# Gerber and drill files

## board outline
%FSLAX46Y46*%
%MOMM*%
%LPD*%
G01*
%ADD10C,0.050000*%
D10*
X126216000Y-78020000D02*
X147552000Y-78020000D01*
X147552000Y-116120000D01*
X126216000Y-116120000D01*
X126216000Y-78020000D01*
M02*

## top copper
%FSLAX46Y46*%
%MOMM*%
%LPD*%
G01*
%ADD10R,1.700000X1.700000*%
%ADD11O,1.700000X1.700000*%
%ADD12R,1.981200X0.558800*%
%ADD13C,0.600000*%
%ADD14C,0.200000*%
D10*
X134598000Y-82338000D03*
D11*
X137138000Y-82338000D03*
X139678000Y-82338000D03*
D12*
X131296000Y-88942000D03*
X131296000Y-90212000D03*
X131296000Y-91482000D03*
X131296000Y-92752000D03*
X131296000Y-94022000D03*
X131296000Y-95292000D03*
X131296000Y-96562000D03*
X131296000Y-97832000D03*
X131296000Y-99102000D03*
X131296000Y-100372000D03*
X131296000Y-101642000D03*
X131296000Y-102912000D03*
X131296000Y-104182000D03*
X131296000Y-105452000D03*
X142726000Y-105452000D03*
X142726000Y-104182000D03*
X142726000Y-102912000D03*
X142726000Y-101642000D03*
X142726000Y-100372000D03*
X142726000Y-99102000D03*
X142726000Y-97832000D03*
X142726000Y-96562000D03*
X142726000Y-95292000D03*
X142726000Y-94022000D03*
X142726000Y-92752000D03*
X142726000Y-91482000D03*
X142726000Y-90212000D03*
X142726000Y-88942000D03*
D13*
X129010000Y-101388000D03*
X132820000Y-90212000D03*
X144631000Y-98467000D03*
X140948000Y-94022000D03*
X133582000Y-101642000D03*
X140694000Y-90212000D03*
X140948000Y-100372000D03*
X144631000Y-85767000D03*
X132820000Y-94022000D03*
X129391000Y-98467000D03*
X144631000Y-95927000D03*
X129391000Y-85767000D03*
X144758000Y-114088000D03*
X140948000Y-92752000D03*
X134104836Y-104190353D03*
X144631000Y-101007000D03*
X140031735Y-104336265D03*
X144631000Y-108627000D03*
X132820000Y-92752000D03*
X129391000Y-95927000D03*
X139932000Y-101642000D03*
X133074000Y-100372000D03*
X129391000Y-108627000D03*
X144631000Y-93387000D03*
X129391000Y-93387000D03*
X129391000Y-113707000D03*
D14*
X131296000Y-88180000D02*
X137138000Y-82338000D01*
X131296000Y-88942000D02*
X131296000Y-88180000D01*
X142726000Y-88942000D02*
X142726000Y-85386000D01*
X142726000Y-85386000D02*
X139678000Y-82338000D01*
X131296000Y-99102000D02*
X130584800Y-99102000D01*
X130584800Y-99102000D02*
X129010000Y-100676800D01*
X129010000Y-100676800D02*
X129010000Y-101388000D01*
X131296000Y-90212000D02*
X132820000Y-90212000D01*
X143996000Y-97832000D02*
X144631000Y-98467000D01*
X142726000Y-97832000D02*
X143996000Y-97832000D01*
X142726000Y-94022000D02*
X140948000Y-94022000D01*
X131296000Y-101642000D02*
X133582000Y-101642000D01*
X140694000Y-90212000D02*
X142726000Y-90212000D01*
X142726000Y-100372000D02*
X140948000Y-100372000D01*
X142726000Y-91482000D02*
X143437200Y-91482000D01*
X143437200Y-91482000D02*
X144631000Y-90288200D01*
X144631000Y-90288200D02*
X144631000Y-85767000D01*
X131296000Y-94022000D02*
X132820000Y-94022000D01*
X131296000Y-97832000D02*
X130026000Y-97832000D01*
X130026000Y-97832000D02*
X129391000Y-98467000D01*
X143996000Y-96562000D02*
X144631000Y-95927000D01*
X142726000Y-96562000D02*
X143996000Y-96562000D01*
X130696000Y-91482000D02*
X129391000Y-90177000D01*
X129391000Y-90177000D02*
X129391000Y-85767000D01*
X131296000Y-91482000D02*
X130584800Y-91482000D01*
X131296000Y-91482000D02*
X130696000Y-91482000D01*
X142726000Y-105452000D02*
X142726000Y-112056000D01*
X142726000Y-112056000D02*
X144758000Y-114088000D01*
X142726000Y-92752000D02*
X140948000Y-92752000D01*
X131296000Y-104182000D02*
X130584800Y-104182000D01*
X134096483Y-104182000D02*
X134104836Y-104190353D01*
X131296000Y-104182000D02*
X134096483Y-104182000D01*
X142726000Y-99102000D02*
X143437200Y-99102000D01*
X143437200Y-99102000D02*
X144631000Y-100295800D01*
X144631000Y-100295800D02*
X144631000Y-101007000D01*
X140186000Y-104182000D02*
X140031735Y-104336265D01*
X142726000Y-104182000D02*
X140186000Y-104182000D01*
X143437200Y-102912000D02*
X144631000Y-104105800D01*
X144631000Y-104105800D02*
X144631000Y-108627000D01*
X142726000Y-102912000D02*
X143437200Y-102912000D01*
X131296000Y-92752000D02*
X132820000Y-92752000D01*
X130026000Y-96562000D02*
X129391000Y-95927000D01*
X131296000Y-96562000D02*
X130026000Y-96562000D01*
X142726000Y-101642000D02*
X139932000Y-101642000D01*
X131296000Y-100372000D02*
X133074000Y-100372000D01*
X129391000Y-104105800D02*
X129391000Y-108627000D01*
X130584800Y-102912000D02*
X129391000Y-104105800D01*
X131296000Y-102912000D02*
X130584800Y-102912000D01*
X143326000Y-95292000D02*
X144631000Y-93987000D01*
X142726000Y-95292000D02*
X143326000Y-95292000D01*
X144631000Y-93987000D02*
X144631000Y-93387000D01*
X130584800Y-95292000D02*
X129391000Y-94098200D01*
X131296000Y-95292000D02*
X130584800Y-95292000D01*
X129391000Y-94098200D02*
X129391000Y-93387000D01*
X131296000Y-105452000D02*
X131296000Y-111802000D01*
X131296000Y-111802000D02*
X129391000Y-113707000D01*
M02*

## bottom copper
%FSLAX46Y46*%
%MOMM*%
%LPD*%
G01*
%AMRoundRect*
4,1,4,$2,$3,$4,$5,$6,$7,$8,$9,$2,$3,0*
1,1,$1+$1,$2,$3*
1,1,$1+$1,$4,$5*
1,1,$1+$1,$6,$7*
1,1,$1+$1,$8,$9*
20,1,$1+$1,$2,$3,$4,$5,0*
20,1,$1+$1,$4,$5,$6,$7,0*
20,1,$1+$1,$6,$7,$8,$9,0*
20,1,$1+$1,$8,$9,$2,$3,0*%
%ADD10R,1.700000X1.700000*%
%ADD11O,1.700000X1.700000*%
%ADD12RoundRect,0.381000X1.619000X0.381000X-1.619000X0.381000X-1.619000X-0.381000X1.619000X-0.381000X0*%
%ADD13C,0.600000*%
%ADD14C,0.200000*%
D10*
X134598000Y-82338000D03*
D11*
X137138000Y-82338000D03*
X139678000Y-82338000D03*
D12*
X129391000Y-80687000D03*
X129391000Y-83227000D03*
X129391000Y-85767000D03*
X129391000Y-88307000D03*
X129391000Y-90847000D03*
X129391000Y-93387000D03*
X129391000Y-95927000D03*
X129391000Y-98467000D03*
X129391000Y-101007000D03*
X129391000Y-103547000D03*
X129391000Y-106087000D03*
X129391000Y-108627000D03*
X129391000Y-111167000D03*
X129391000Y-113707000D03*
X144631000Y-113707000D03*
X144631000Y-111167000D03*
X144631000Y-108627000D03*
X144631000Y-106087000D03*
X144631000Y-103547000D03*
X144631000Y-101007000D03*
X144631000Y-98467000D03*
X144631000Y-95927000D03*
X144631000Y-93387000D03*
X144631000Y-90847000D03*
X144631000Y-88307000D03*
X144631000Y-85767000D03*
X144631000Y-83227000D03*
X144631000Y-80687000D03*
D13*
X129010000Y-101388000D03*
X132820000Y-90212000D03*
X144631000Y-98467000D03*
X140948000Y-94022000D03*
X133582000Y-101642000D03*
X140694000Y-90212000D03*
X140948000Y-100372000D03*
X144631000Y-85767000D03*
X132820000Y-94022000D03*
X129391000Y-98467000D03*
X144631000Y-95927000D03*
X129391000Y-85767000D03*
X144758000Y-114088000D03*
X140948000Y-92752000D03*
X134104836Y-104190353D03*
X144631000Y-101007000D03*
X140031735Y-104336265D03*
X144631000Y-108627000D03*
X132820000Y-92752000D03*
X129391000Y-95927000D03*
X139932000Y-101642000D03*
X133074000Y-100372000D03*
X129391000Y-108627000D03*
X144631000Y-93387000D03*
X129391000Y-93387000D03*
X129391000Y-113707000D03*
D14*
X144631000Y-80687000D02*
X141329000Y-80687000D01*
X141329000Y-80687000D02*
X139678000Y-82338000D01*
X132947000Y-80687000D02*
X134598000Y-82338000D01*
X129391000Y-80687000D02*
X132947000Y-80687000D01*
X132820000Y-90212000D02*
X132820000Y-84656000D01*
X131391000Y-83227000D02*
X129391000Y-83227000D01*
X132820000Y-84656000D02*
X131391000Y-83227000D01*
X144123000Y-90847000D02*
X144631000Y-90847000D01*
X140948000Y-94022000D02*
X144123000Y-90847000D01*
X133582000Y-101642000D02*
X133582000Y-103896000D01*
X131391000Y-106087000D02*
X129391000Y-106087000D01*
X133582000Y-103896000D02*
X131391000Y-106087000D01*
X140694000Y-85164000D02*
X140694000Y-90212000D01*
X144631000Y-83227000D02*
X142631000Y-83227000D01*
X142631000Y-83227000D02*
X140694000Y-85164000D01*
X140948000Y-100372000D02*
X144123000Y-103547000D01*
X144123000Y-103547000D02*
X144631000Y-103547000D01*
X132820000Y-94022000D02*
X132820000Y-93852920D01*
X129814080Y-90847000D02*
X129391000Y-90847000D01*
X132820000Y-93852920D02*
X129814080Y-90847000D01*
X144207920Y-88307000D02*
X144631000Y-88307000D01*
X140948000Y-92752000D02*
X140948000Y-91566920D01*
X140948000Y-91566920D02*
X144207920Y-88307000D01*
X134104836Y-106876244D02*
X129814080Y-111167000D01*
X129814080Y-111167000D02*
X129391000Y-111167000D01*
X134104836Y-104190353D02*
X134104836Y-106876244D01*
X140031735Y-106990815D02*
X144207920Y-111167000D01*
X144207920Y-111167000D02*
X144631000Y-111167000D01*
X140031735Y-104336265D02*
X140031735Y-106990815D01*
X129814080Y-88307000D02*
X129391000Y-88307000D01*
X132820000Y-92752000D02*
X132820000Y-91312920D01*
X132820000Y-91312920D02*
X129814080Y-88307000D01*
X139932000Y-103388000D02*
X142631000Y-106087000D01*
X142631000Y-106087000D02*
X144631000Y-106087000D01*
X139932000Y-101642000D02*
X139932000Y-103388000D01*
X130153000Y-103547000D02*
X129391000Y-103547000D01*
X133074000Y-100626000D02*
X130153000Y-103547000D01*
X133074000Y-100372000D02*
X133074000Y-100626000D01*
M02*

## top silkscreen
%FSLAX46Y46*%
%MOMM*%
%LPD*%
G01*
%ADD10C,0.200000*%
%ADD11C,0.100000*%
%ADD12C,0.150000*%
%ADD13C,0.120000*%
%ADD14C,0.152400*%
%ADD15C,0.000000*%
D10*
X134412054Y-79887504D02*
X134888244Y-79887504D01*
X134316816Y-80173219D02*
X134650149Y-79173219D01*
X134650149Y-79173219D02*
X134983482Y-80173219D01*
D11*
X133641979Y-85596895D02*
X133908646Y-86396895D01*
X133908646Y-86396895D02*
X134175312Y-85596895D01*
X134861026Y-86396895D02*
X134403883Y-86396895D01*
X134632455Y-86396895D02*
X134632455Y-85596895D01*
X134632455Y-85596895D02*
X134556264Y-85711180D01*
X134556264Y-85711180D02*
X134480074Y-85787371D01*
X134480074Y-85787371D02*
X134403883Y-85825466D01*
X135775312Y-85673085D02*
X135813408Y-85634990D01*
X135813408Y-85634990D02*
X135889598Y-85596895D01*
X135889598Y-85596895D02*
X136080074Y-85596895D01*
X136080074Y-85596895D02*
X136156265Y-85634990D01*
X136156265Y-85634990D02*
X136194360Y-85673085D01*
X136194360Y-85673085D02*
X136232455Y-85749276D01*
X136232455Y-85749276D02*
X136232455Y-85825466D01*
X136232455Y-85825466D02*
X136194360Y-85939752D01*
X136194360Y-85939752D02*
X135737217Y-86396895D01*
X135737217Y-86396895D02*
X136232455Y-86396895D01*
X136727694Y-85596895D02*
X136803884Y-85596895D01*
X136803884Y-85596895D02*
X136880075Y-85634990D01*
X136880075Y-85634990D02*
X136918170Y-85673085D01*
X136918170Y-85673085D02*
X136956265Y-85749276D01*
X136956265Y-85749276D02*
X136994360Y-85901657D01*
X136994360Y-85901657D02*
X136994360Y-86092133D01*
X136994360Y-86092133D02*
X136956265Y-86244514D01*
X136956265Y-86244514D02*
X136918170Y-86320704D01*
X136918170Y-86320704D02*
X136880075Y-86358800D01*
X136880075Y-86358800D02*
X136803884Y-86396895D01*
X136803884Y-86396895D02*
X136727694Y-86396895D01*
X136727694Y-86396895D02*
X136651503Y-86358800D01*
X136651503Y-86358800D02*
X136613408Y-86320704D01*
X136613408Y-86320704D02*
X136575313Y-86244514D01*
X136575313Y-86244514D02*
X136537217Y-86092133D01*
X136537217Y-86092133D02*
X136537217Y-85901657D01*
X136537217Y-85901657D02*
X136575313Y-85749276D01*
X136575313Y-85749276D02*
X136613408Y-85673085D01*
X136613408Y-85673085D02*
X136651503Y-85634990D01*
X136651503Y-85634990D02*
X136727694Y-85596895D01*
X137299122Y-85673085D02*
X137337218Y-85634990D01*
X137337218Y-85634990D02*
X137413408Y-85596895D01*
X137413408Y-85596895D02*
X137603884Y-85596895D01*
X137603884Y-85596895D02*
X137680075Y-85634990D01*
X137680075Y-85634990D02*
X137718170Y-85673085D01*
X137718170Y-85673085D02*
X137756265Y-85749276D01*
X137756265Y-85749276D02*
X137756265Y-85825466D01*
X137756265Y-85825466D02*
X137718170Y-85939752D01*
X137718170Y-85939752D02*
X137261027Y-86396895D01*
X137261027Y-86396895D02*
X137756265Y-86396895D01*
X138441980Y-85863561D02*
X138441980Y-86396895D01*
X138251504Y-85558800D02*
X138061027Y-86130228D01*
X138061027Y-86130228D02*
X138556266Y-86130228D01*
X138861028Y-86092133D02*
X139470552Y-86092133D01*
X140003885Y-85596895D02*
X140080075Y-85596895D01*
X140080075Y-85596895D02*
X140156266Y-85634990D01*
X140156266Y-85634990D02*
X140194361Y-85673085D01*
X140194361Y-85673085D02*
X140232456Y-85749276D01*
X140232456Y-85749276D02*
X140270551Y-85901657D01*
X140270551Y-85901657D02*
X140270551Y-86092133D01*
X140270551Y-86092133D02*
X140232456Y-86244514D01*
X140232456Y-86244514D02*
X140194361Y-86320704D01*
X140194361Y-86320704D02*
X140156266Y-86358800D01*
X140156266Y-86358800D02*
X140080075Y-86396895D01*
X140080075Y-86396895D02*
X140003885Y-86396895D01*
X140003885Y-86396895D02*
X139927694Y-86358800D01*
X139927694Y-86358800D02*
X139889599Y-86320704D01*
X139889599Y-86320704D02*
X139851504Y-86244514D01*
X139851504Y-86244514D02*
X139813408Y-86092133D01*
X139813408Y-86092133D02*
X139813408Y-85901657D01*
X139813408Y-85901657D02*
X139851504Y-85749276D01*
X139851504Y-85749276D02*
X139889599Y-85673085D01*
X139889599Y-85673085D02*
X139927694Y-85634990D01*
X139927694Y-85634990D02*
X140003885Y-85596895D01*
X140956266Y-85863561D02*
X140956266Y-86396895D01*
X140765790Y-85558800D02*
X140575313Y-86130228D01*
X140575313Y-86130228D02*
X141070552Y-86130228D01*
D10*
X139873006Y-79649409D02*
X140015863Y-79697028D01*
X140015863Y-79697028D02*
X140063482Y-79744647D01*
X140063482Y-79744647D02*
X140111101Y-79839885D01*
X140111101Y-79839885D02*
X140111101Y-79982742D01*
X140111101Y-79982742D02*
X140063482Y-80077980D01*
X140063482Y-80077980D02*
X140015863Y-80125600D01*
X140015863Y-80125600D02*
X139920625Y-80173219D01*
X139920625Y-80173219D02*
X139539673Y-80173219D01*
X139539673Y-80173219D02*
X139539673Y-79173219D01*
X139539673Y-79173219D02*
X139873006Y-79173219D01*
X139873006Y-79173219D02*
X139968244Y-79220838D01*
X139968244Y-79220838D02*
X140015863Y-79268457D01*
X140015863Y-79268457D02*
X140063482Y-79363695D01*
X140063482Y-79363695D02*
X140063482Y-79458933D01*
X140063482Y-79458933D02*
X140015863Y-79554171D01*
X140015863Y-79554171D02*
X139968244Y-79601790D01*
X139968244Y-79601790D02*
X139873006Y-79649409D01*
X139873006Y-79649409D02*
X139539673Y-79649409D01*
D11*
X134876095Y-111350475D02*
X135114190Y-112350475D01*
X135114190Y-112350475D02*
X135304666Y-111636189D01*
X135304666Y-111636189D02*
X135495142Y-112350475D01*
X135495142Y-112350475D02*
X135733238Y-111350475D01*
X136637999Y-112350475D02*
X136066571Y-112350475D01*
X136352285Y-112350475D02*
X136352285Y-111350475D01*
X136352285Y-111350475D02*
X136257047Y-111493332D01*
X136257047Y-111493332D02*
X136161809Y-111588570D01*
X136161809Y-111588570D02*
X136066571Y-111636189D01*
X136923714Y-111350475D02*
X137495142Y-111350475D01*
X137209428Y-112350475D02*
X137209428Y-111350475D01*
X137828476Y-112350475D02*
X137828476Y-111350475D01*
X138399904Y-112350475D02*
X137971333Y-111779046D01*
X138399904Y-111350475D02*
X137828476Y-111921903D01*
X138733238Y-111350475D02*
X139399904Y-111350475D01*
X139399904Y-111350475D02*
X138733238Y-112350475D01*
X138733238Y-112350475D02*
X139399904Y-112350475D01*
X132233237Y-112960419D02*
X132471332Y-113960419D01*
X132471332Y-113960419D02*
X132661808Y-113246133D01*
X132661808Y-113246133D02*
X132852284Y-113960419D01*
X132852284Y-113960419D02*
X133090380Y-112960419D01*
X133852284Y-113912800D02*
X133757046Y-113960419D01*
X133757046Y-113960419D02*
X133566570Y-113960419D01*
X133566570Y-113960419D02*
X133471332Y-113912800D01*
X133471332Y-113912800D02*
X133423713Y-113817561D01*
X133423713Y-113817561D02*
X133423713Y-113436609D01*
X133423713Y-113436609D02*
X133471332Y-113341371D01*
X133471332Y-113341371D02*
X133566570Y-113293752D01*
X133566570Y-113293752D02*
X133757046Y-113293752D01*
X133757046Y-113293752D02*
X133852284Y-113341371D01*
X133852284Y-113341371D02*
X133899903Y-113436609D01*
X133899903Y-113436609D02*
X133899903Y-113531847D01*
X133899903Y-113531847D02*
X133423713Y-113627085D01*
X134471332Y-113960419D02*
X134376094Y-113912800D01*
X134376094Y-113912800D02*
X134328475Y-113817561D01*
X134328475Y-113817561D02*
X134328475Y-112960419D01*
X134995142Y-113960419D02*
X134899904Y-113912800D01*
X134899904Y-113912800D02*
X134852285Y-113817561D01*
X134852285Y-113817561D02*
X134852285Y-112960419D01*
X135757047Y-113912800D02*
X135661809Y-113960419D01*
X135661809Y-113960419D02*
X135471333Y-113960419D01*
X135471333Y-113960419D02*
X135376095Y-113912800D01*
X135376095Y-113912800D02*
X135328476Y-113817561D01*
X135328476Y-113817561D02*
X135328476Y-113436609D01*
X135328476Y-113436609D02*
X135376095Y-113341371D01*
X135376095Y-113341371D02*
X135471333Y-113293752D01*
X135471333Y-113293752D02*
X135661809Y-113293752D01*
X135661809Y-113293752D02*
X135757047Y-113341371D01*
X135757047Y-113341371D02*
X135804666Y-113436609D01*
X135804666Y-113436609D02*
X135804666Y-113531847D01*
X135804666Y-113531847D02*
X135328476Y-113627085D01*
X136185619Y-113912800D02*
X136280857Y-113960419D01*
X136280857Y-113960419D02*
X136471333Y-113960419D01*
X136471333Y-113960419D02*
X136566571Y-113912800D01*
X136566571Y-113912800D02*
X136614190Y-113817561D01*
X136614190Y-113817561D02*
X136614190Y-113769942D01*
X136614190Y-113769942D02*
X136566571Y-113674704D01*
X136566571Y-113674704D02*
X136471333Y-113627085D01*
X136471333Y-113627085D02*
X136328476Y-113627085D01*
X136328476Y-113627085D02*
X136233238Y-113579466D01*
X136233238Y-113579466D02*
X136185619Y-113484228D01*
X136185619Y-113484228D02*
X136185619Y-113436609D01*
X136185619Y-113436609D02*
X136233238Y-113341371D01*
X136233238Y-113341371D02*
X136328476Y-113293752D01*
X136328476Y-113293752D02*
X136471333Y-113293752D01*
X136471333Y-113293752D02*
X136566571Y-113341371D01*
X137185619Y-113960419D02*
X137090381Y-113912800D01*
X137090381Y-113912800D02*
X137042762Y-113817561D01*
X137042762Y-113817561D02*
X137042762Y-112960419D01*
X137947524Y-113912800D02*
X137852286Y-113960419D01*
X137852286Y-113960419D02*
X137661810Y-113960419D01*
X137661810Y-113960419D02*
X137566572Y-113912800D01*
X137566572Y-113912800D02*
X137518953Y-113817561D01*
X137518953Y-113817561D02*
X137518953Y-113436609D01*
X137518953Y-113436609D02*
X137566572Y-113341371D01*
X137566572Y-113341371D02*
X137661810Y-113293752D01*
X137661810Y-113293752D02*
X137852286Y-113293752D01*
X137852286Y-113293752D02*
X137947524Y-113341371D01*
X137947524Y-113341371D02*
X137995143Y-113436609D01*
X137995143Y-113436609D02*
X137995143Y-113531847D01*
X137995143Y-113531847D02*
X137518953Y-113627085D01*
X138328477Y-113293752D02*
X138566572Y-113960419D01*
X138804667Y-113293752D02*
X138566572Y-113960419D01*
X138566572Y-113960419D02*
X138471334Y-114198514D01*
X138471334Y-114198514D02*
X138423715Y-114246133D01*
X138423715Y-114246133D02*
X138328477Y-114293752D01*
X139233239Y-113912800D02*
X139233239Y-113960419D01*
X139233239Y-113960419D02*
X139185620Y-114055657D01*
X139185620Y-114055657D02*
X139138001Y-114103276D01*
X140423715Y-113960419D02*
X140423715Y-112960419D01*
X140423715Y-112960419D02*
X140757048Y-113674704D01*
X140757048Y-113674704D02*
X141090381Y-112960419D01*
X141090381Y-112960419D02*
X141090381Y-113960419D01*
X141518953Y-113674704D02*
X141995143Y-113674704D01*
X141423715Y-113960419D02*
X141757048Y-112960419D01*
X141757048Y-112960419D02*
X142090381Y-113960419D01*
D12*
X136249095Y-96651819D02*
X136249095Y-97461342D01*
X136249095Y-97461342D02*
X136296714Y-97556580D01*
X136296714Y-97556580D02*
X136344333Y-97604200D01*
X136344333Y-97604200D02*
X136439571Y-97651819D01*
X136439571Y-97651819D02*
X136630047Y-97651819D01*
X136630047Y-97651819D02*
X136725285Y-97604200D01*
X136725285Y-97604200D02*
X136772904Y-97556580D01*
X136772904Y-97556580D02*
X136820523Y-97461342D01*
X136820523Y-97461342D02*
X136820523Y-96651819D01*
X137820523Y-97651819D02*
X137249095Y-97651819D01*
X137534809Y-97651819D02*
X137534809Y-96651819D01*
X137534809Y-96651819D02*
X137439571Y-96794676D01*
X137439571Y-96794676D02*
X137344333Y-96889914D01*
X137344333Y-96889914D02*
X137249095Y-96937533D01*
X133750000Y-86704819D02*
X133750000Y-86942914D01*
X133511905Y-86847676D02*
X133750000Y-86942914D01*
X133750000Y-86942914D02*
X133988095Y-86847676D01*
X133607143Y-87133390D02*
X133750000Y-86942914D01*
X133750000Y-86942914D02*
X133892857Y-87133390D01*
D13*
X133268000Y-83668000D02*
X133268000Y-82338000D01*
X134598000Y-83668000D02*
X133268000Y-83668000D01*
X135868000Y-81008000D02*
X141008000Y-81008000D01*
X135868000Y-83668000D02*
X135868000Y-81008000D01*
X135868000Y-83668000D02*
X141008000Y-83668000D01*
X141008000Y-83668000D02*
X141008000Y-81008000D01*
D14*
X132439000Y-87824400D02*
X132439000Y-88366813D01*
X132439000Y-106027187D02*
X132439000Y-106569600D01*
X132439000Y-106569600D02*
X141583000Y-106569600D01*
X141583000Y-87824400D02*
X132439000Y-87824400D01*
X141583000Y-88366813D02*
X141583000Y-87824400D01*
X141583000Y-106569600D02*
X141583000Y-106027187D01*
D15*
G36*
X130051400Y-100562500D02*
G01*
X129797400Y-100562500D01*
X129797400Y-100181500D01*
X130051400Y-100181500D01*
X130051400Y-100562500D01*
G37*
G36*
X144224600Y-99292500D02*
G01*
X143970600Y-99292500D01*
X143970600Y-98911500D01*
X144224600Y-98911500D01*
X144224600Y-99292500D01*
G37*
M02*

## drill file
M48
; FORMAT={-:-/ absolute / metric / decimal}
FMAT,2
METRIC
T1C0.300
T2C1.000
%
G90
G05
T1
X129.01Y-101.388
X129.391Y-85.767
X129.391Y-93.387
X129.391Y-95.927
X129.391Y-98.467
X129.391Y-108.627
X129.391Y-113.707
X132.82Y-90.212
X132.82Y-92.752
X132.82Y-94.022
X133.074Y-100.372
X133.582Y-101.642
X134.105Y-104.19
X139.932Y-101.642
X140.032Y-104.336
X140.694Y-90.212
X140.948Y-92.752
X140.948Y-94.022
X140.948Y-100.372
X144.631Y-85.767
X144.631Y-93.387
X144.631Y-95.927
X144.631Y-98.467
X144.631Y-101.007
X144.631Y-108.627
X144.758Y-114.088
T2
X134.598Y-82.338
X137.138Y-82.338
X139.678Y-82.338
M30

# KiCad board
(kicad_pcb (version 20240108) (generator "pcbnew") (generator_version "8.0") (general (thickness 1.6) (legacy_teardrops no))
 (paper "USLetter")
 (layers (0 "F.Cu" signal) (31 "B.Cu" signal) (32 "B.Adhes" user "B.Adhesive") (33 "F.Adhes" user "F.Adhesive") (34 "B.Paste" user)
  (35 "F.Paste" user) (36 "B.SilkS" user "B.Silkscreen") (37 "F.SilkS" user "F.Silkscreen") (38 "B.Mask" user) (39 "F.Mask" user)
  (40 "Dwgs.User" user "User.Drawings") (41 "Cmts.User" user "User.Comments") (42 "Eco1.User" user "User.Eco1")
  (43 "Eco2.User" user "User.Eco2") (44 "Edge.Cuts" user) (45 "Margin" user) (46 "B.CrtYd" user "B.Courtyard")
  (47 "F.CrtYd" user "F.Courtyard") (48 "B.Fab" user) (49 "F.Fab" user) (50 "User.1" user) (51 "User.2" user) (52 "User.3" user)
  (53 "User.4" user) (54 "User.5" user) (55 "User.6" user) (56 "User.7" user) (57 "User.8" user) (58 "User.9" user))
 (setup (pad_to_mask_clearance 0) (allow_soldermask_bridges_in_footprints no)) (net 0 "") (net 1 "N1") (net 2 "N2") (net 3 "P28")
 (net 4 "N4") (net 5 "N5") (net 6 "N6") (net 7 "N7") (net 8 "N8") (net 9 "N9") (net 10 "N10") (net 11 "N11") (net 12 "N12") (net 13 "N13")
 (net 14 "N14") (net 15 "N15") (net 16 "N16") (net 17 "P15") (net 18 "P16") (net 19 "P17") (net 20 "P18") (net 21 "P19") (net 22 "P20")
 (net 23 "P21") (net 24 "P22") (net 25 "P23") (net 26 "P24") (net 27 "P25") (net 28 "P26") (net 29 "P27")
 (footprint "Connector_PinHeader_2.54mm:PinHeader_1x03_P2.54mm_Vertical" (layer "F.Cu") (at 134.598 82.338 90)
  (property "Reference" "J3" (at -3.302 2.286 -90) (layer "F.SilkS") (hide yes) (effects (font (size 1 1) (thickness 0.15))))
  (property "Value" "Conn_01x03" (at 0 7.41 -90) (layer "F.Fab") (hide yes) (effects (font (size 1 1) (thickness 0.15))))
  (fp_line (start -1.33 -1.33) (end 0 -1.33) (stroke (width 0.12) (type solid)) (layer "F.SilkS"))
  (fp_line (start -1.33 0) (end -1.33 -1.33) (stroke (width 0.12) (type solid)) (layer "F.SilkS"))
  (fp_line (start 1.33 1.27) (end 1.33 6.41) (stroke (width 0.12) (type solid)) (layer "F.SilkS"))
  (fp_line (start -1.33 1.27) (end 1.33 1.27) (stroke (width 0.12) (type solid)) (layer "F.SilkS"))
  (fp_line (start -1.33 1.27) (end -1.33 6.41) (stroke (width 0.12) (type solid)) (layer "F.SilkS"))
  (fp_line (start -1.33 6.41) (end 1.33 6.41) (stroke (width 0.12) (type solid)) (layer "F.SilkS"))
  (pad "1" thru_hole rect (at 0 0 90) (size 1.7 1.7) (drill 1) (layers "*.Cu" "*.Mask") (remove_unused_layers no) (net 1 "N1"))
  (pad "2" thru_hole oval (at 0 2.54 90) (size 1.7 1.7) (drill 1) (layers "*.Cu" "*.Mask") (remove_unused_layers no) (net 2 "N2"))
  (pad "3" thru_hole oval (at 0 5.08 90) (size 1.7 1.7) (drill 1) (layers "*.Cu" "*.Mask") (remove_unused_layers no) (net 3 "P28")))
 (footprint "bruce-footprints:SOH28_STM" (layer "F.Cu") (at 137.011 97.197)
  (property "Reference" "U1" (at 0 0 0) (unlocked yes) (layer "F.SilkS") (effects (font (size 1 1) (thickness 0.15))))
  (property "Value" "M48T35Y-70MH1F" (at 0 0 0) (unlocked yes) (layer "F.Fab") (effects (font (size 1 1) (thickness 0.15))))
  (fp_line (start -4.572 -9.3726) (end -4.572 -8.830187) (stroke (width 0.1524) (type solid)) (layer "F.SilkS"))
  (fp_line (start -4.572 8.830187) (end -4.572 9.3726) (stroke (width 0.1524) (type solid)) (layer "F.SilkS"))
  (fp_line (start -4.572 9.3726) (end 4.572 9.3726) (stroke (width 0.1524) (type solid)) (layer "F.SilkS"))
  (fp_line (start 4.572 -9.3726) (end -4.572 -9.3726) (stroke (width 0.1524) (type solid)) (layer "F.SilkS"))
  (fp_line (start 4.572 -8.830187) (end 4.572 -9.3726) (stroke (width 0.1524) (type solid)) (layer "F.SilkS"))
  (fp_line (start 4.572 9.3726) (end 4.572 8.830187) (stroke (width 0.1524) (type solid)) (layer "F.SilkS"))
  (fp_poly
   (pts (xy -7.2136 2.9845) (xy -7.2136 3.3655) (xy -6.9596 3.3655) (xy -6.9596 2.9845)) (stroke (width 0) (type solid)) (fill solid)
   (layer "F.SilkS"))
  (fp_poly
   (pts (xy 7.2136 1.7145) (xy 7.2136 2.0955) (xy 6.9596 2.0955) (xy 6.9596 1.7145)) (stroke (width 0) (type solid)) (fill solid)
   (layer "F.SilkS"))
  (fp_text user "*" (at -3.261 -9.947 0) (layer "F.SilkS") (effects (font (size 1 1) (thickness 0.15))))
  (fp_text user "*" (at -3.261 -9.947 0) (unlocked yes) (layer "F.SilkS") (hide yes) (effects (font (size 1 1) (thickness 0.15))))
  (pad "1" smd rect (at -5.715 -8.255) (size 1.9812 0.5588) (layers "F.Cu" "F.Paste" "F.Mask") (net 2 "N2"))
  (pad "2" smd rect (at -5.715 -6.985) (size 1.9812 0.5588) (layers "F.Cu" "F.Paste" "F.Mask") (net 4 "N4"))
  (pad "3" smd rect (at -5.715 -5.715) (size 1.9812 0.5588) (layers "F.Cu" "F.Paste" "F.Mask") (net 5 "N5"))
  (pad "4" smd rect (at -5.715 -4.445) (size 1.9812 0.5588) (layers "F.Cu" "F.Paste" "F.Mask") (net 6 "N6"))
  (pad "5" smd rect (at -5.715 -3.175) (size 1.9812 0.5588) (layers "F.Cu" "F.Paste" "F.Mask") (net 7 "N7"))
  (pad "6" smd rect (at -5.715 -1.905) (size 1.9812 0.5588) (layers "F.Cu" "F.Paste" "F.Mask") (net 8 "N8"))
  (pad "7" smd rect (at -5.715 -0.635) (size 1.9812 0.5588) (layers "F.Cu" "F.Paste" "F.Mask") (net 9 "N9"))
  (pad "8" smd rect (at -5.715 0.635) (size 1.9812 0.5588) (layers "F.Cu" "F.Paste" "F.Mask") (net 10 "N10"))
  (pad "9" smd rect (at -5.715 1.905) (size 1.9812 0.5588) (layers "F.Cu" "F.Paste" "F.Mask") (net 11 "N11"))
  (pad "10" smd rect (at -5.715 3.175) (size 1.9812 0.5588) (layers "F.Cu" "F.Paste" "F.Mask") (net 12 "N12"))
  (pad "11" smd rect (at -5.715 4.445) (size 1.9812 0.5588) (layers "F.Cu" "F.Paste" "F.Mask") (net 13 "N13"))
  (pad "12" smd rect (at -5.715 5.715) (size 1.9812 0.5588) (layers "F.Cu" "F.Paste" "F.Mask") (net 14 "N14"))
  (pad "13" smd rect (at -5.715 6.985) (size 1.9812 0.5588) (layers "F.Cu" "F.Paste" "F.Mask") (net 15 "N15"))
  (pad "14" smd rect (at -5.715 8.255) (size 1.9812 0.5588) (layers "F.Cu" "F.Paste" "F.Mask") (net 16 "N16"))
  (pad "15" smd rect (at 5.715 8.255) (size 1.9812 0.5588) (layers "F.Cu" "F.Paste" "F.Mask") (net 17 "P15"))
  (pad "16" smd rect (at 5.715 6.985) (size 1.9812 0.5588) (layers "F.Cu" "F.Paste" "F.Mask") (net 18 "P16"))
  (pad "17" smd rect (at 5.715 5.715) (size 1.9812 0.5588) (layers "F.Cu" "F.Paste" "F.Mask") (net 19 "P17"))
  (pad "18" smd rect (at 5.715 4.445) (size 1.9812 0.5588) (layers "F.Cu" "F.Paste" "F.Mask") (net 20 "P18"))
  (pad "19" smd rect (at 5.715 3.175) (size 1.9812 0.5588) (layers "F.Cu" "F.Paste" "F.Mask") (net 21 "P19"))
  (pad "20" smd rect (at 5.715 1.905) (size 1.9812 0.5588) (layers "F.Cu" "F.Paste" "F.Mask") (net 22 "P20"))
  (pad "21" smd rect (at 5.715 0.635) (size 1.9812 0.5588) (layers "F.Cu" "F.Paste" "F.Mask") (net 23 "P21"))
  (pad "22" smd rect (at 5.715 -0.635) (size 1.9812 0.5588) (layers "F.Cu" "F.Paste" "F.Mask") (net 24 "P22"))
  (pad "23" smd rect (at 5.715 -1.905) (size 1.9812 0.5588) (layers "F.Cu" "F.Paste" "F.Mask") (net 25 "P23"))
  (pad "24" smd rect (at 5.715 -3.175) (size 1.9812 0.5588) (layers "F.Cu" "F.Paste" "F.Mask") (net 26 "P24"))
  (pad "25" smd rect (at 5.715 -4.445) (size 1.9812 0.5588) (layers "F.Cu" "F.Paste" "F.Mask") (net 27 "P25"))
  (pad "26" smd rect (at 5.715 -5.715) (size 1.9812 0.5588) (layers "F.Cu" "F.Paste" "F.Mask") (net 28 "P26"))
  (pad "27" smd rect (at 5.715 -6.985) (size 1.9812 0.5588) (layers "F.Cu" "F.Paste" "F.Mask") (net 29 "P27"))
  (pad "28" smd rect (at 5.715 -8.255) (size 1.9812 0.5588) (layers "F.Cu" "F.Paste" "F.Mask") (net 3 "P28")))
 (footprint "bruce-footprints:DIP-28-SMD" (layer "B.Cu") (at 137.011 90.847 180)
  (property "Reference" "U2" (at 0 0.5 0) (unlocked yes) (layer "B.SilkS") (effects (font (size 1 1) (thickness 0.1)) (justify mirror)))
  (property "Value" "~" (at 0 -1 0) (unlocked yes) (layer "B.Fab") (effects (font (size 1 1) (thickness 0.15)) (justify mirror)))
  (pad "1" smd roundrect (at 7.62 10.16 180) (size 4 1.524) (layers "B.Cu" "B.Paste" "B.Mask") (roundrect_rratio 0.25) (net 1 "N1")
   (thermal_bridge_angle 45))
  (pad "2" smd roundrect (at 7.62 7.62 180) (size 4 1.524) (layers "B.Cu" "B.Paste" "B.Mask") (roundrect_rratio 0.25) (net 4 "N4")
   (thermal_bridge_angle 45))
  (pad "3" smd roundrect (at 7.62 5.08 180) (size 4 1.524) (layers "B.Cu" "B.Paste" "B.Mask") (roundrect_rratio 0.25) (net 5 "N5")
   (thermal_bridge_angle 45))
  (pad "4" smd roundrect (at 7.62 2.54 180) (size 4 1.524) (layers "B.Cu" "B.Paste" "B.Mask") (roundrect_rratio 0.25) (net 6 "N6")
   (thermal_bridge_angle 45))
  (pad "5" smd roundrect (at 7.62 0 180) (size 4 1.524) (layers "B.Cu" "B.Paste" "B.Mask") (roundrect_rratio 0.25) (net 7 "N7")
   (thermal_bridge_angle 45))
  (pad "6" smd roundrect (at 7.62 -2.54 180) (size 4 1.524) (layers "B.Cu" "B.Paste" "B.Mask") (roundrect_rratio 0.25) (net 8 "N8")
   (thermal_bridge_angle 45))
  (pad "7" smd roundrect (at 7.62 -5.08 180) (size 4 1.524) (layers "B.Cu" "B.Paste" "B.Mask") (roundrect_rratio 0.25) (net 9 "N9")
   (thermal_bridge_angle 45))
  (pad "8" smd roundrect (at 7.62 -7.62 180) (size 4 1.524) (layers "B.Cu" "B.Paste" "B.Mask") (roundrect_rratio 0.25) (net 10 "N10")
   (thermal_bridge_angle 45))
  (pad "9" smd roundrect (at 7.62 -10.16 180) (size 4 1.524) (layers "B.Cu" "B.Paste" "B.Mask") (roundrect_rratio 0.25) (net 11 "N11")
   (thermal_bridge_angle 45))
  (pad "10" smd roundrect (at 7.62 -12.7 180) (size 4 1.524) (layers "B.Cu" "B.Paste" "B.Mask") (roundrect_rratio 0.25) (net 12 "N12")
   (thermal_bridge_angle 45))
  (pad "11" smd roundrect (at 7.62 -15.24 180) (size 4 1.524) (layers "B.Cu" "B.Paste" "B.Mask") (roundrect_rratio 0.25) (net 13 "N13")
   (thermal_bridge_angle 45))
  (pad "12" smd roundrect (at 7.62 -17.78 180) (size 4 1.524) (layers "B.Cu" "B.Paste" "B.Mask") (roundrect_rratio 0.25) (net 14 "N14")
   (thermal_bridge_angle 45))
  (pad "13" smd roundrect (at 7.62 -20.32 180) (size 4 1.524) (layers "B.Cu" "B.Paste" "B.Mask") (roundrect_rratio 0.25) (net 15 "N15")
   (thermal_bridge_angle 45))
  (pad "14" smd roundrect (at 7.62 -22.86 180) (size 4 1.524) (layers "B.Cu" "B.Paste" "B.Mask") (roundrect_rratio 0.25) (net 16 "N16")
   (thermal_bridge_angle 45))
  (pad "15" smd roundrect (at -7.62 -22.86 180) (size 4 1.524) (layers "B.Cu" "B.Paste" "B.Mask") (roundrect_rratio 0.25) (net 17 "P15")
   (thermal_bridge_angle 45))
  (pad "16" smd roundrect (at -7.62 -20.32 180) (size 4 1.524) (layers "B.Cu" "B.Paste" "B.Mask") (roundrect_rratio 0.25) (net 18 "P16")
   (thermal_bridge_angle 45))
  (pad "17" smd roundrect (at -7.62 -17.78 180) (size 4 1.524) (layers "B.Cu" "B.Paste" "B.Mask") (roundrect_rratio 0.25) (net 19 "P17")
   (thermal_bridge_angle 45))
  (pad "18" smd roundrect (at -7.62 -15.24 180) (size 4 1.524) (layers "B.Cu" "B.Paste" "B.Mask") (roundrect_rratio 0.25) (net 20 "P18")
   (thermal_bridge_angle 45))
  (pad "19" smd roundrect (at -7.62 -12.7 180) (size 4 1.524) (layers "B.Cu" "B.Paste" "B.Mask") (roundrect_rratio 0.25) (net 21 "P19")
   (thermal_bridge_angle 45))
  (pad "20" smd roundrect (at -7.62 -10.16 180) (size 4 1.524) (layers "B.Cu" "B.Paste" "B.Mask") (roundrect_rratio 0.25) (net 22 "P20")
   (thermal_bridge_angle 45))
  (pad "21" smd roundrect (at -7.62 -7.62 180) (size 4 1.524) (layers "B.Cu" "B.Paste" "B.Mask") (roundrect_rratio 0.25) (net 23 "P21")
   (thermal_bridge_angle 45))
  (pad "22" smd roundrect (at -7.62 -5.08 180) (size 4 1.524) (layers "B.Cu" "B.Paste" "B.Mask") (roundrect_rratio 0.25) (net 24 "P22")
   (thermal_bridge_angle 45))
  (pad "23" smd roundrect (at -7.62 -2.54 180) (size 4 1.524) (layers "B.Cu" "B.Paste" "B.Mask") (roundrect_rratio 0.25) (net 25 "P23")
   (thermal_bridge_angle 45))
  (pad "24" smd roundrect (at -7.62 0 180) (size 4 1.524) (layers "B.Cu" "B.Paste" "B.Mask") (roundrect_rratio 0.25) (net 26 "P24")
   (thermal_bridge_angle 45))
  (pad "25" smd roundrect (at -7.62 2.54 180) (size 4 1.524) (layers "B.Cu" "B.Paste" "B.Mask") (roundrect_rratio 0.25) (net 27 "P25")
   (thermal_bridge_angle 45))
  (pad "26" smd roundrect (at -7.62 5.08 180) (size 4 1.524) (layers "B.Cu" "B.Paste" "B.Mask") (roundrect_rratio 0.25) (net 28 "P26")
   (thermal_bridge_angle 45))
  (pad "27" smd roundrect (at -7.62 7.62 180) (size 4 1.524) (layers "B.Cu" "B.Paste" "B.Mask") (roundrect_rratio 0.25) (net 29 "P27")
   (thermal_bridge_angle 45))
  (pad "28" smd roundrect (at -7.62 10.16 180) (size 4 1.524) (layers "B.Cu" "B.Paste" "B.Mask") (roundrect_rratio 0.25) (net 3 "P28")
   (thermal_bridge_angle 45)))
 (gr_rect (start 126.216 78.02) (end 147.552 116.12) (stroke (width 0.05) (type default)) (fill none) (layer "Edge.Cuts"))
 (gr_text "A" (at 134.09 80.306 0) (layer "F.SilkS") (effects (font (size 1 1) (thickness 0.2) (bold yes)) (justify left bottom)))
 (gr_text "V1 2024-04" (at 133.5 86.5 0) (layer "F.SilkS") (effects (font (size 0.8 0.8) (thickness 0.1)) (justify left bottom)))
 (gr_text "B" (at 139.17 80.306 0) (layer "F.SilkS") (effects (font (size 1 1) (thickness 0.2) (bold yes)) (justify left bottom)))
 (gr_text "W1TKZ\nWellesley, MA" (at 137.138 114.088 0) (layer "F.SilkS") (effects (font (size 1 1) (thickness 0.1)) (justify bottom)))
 (segment (start 131.296 88.18) (end 137.138 82.338) (width 0.2) (layer "F.Cu") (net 2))
 (segment (start 131.296 88.942) (end 131.296 88.18) (width 0.2) (layer "F.Cu") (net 2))
 (segment (start 142.726 88.942) (end 142.726 85.386) (width 0.2) (layer "F.Cu") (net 3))
 (segment (start 142.726 85.386) (end 139.678 82.338) (width 0.2) (layer "F.Cu") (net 3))
 (segment (start 144.631 80.687) (end 141.329 80.687) (width 0.2) (layer "B.Cu") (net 3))
 (segment (start 141.329 80.687) (end 139.678 82.338) (width 0.2) (layer "B.Cu") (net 3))
 (segment (start 132.947 80.687) (end 134.598 82.338) (width 0.2) (layer "B.Cu") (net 1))
 (segment (start 129.391 80.687) (end 132.947 80.687) (width 0.2) (layer "B.Cu") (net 1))
 (segment (start 131.296 99.102) (end 130.5848 99.102) (width 0.2) (layer "F.Cu") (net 11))
 (segment (start 130.5848 99.102) (end 129.01 100.6768) (width 0.2) (layer "F.Cu") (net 11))
 (segment (start 129.01 100.6768) (end 129.01 101.388) (width 0.2) (layer "F.Cu") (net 11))
 (via (at 129.01 101.388) (size 0.6) (drill 0.3) (layers "F.Cu" "B.Cu") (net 11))
 (segment (start 131.296 90.212) (end 132.82 90.212) (width 0.2) (layer "F.Cu") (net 4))
 (via (at 132.82 90.212) (size 0.6) (drill 0.3) (layers "F.Cu" "B.Cu") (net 4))
 (segment (start 132.82 90.212) (end 132.82 84.656) (width 0.2) (layer "B.Cu") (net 4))
 (segment (start 131.391 83.227) (end 129.391 83.227) (width 0.2) (layer "B.Cu") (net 4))
 (segment (start 132.82 84.656) (end 131.391 83.227) (width 0.2) (layer "B.Cu") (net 4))
 (segment (start 143.996 97.832) (end 144.631 98.467) (width 0.2) (layer "F.Cu") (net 23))
 (segment (start 142.726 97.832) (end 143.996 97.832) (width 0.2) (layer "F.Cu") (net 23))
 (via (at 144.631 98.467) (size 0.6) (drill 0.3) (layers "F.Cu" "B.Cu") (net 23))
 (segment (start 142.726 94.022) (end 140.948 94.022) (width 0.2) (layer "F.Cu") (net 26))
 (via (at 140.948 94.022) (size 0.6) (drill 0.3) (layers "F.Cu" "B.Cu") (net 26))
 (segment (start 144.123 90.847) (end 144.631 90.847) (width 0.2) (layer "B.Cu") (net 26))
 (segment (start 140.948 94.022) (end 144.123 90.847) (width 0.2) (layer "B.Cu") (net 26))
 (segment (start 131.296 101.642) (end 133.582 101.642) (width 0.2) (layer "F.Cu") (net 13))
 (via (at 133.582 101.642) (size 0.6) (drill 0.3) (layers "F.Cu" "B.Cu") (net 13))
 (segment (start 133.582 101.642) (end 133.582 103.896) (width 0.2) (layer "B.Cu") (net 13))
 (segment (start 131.391 106.087) (end 129.391 106.087) (width 0.2) (layer "B.Cu") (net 13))
 (segment (start 133.582 103.896) (end 131.391 106.087) (width 0.2) (layer "B.Cu") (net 13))
 (segment (start 140.694 90.212) (end 142.726 90.212) (width 0.2) (layer "F.Cu") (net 29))
 (via (at 140.694 90.212) (size 0.6) (drill 0.3) (layers "F.Cu" "B.Cu") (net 29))
 (segment (start 140.694 85.164) (end 140.694 90.212) (width 0.2) (layer "B.Cu") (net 29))
 (segment (start 144.631 83.227) (end 142.631 83.227) (width 0.2) (layer "B.Cu") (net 29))
 (segment (start 142.631 83.227) (end 140.694 85.164) (width 0.2) (layer "B.Cu") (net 29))
 (segment (start 142.726 100.372) (end 140.948 100.372) (width 0.2) (layer "F.Cu") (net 21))
 (via (at 140.948 100.372) (size 0.6) (drill 0.3) (layers "F.Cu" "B.Cu") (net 21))
 (segment (start 140.948 100.372) (end 144.123 103.547) (width 0.2) (layer "B.Cu") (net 21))
 (segment (start 144.123 103.547) (end 144.631 103.547) (width 0.2) (layer "B.Cu") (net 21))
 (segment (start 142.726 91.482) (end 143.4372 91.482) (width 0.2) (layer "F.Cu") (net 28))
 (segment (start 143.4372 91.482) (end 144.631 90.2882) (width 0.2) (layer "F.Cu") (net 28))
 (segment (start 144.631 90.2882) (end 144.631 85.767) (width 0.2) (layer "F.Cu") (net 28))
 (via (at 144.631 85.767) (size 0.6) (drill 0.3) (layers "F.Cu" "B.Cu") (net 28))
 (segment (start 131.296 94.022) (end 132.82 94.022) (width 0.2) (layer "F.Cu") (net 7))
 (via (at 132.82 94.022) (size 0.6) (drill 0.3) (layers "F.Cu" "B.Cu") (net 7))
 (segment (start 132.82 94.022) (end 132.82 93.85292) (width 0.2) (layer "B.Cu") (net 7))
 (segment (start 129.81408 90.847) (end 129.391 90.847) (width 0.2) (layer "B.Cu") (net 7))
 (segment (start 132.82 93.85292) (end 129.81408 90.847) (width 0.2) (layer "B.Cu") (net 7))
 (segment (start 131.296 97.832) (end 130.026 97.832) (width 0.2) (layer "F.Cu") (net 10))
 (segment (start 130.026 97.832) (end 129.391 98.467) (width 0.2) (layer "F.Cu") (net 10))
 (via (at 129.391 98.467) (size 0.6) (drill 0.3) (layers "F.Cu" "B.Cu") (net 10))
 (segment (start 143.996 96.562) (end 144.631 95.927) (width 0.2) (layer "F.Cu") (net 24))
 (segment (start 142.726 96.562) (end 143.996 96.562) (width 0.2) (layer "F.Cu") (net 24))
 (via (at 144.631 95.927) (size 0.6) (drill 0.3) (layers "F.Cu" "B.Cu") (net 24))
 (segment (start 130.696 91.482) (end 129.391 90.177) (width 0.2) (layer "F.Cu") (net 5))
 (segment (start 129.391 90.177) (end 129.391 85.767) (width 0.2) (layer "F.Cu") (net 5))
 (segment (start 131.296 91.482) (end 130.5848 91.482) (width 0.2) (layer "F.Cu") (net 5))
 (segment (start 131.296 91.482) (end 130.696 91.482) (width 0.2) (layer "F.Cu") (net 5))
 (via (at 129.391 85.767) (size 0.6) (drill 0.3) (layers "F.Cu" "B.Cu") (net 5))
 (segment (start 142.726 105.452) (end 142.726 112.056) (width 0.2) (layer "F.Cu") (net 17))
 (segment (start 142.726 112.056) (end 144.758 114.088) (width 0.2) (layer "F.Cu") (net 17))
 (via (at 144.758 114.088) (size 0.6) (drill 0.3) (layers "F.Cu" "B.Cu") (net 17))
 (segment (start 142.726 92.752) (end 140.948 92.752) (width 0.2) (layer "F.Cu") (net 27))
 (via (at 140.948 92.752) (size 0.6) (drill 0.3) (layers "F.Cu" "B.Cu") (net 27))
 (segment (start 144.20792 88.307) (end 144.631 88.307) (width 0.2) (layer "B.Cu") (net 27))
 (segment (start 140.948 92.752) (end 140.948 91.56692) (width 0.2) (layer "B.Cu") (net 27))
 (segment (start 140.948 91.56692) (end 144.20792 88.307) (width 0.2) (layer "B.Cu") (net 27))
 (segment (start 131.296 104.182) (end 130.5848 104.182) (width 0.2) (layer "F.Cu") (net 15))
 (segment (start 134.096483 104.182) (end 134.104836 104.190353) (width 0.2) (layer "F.Cu") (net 15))
 (segment (start 131.296 104.182) (end 134.096483 104.182) (width 0.2) (layer "F.Cu") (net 15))
 (via (at 134.104836 104.190353) (size 0.6) (drill 0.3) (layers "F.Cu" "B.Cu") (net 15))
 (segment (start 134.104836 106.876244) (end 129.81408 111.167) (width 0.2) (layer "B.Cu") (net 15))
 (segment (start 129.81408 111.167) (end 129.391 111.167) (width 0.2) (layer "B.Cu") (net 15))
 (segment (start 134.104836 104.190353) (end 134.104836 106.876244) (width 0.2) (layer "B.Cu") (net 15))
 (segment (start 142.726 99.102) (end 143.4372 99.102) (width 0.2) (layer "F.Cu") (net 22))
 (segment (start 143.4372 99.102) (end 144.631 100.2958) (width 0.2) (layer "F.Cu") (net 22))
 (segment (start 144.631 100.2958) (end 144.631 101.007) (width 0.2) (layer "F.Cu") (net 22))
 (via (at 144.631 101.007) (size 0.6) (drill 0.3) (layers "F.Cu" "B.Cu") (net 22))
 (segment (start 140.186 104.182) (end 140.031735 104.336265) (width 0.2) (layer "F.Cu") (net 18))
 (segment (start 142.726 104.182) (end 140.186 104.182) (width 0.2) (layer "F.Cu") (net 18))
 (via (at 140.031735 104.336265) (size 0.6) (drill 0.3) (layers "F.Cu" "B.Cu") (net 18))
 (segment (start 140.031735 106.990815) (end 144.20792 111.167) (width 0.2) (layer "B.Cu") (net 18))
 (segment (start 144.20792 111.167) (end 144.631 111.167) (width 0.2) (layer "B.Cu") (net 18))
 (segment (start 140.031735 104.336265) (end 140.031735 106.990815) (width 0.2) (layer "B.Cu") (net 18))
 (segment (start 143.4372 102.912) (end 144.631 104.1058) (width 0.2) (layer "F.Cu") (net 19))
 (segment (start 144.631 104.1058) (end 144.631 108.627) (width 0.2) (layer "F.Cu") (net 19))
 (segment (start 142.726 102.912) (end 143.4372 102.912) (width 0.2) (layer "F.Cu") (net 19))
 (via (at 144.631 108.627) (size 0.6) (drill 0.3) (layers "F.Cu" "B.Cu") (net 19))
 (segment (start 131.296 92.752) (end 132.82 92.752) (width 0.2) (layer "F.Cu") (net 6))
 (via (at 132.82 92.752) (size 0.6) (drill 0.3) (layers "F.Cu" "B.Cu") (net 6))
 (segment (start 129.81408 88.307) (end 129.391 88.307) (width 0.2) (layer "B.Cu") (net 6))
 (segment (start 132.82 92.752) (end 132.82 91.31292) (width 0.2) (layer "B.Cu") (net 6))
 (segment (start 132.82 91.31292) (end 129.81408 88.307) (width 0.2) (layer "B.Cu") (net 6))
 (segment (start 130.026 96.562) (end 129.391 95.927) (width 0.2) (layer "F.Cu") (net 9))
 (segment (start 131.296 96.562) (end 130.026 96.562) (width 0.2) (layer "F.Cu") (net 9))
 (via (at 129.391 95.927) (size 0.6) (drill 0.3) (layers "F.Cu" "B.Cu") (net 9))
 (segment (start 142.726 101.642) (end 139.932 101.642) (width 0.2) (layer "F.Cu") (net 20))
 (via (at 139.932 101.642) (size 0.6) (drill 0.3) (layers "F.Cu" "B.Cu") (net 20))
 (segment (start 139.932 103.388) (end 142.631 106.087) (width 0.2) (layer "B.Cu") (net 20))
 (segment (start 142.631 106.087) (end 144.631 106.087) (width 0.2) (layer "B.Cu") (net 20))
 (segment (start 139.932 101.642) (end 139.932 103.388) (width 0.2) (layer "B.Cu") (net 20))
 (segment (start 131.296 100.372) (end 133.074 100.372) (width 0.2) (layer "F.Cu") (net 12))
 (via (at 133.074 100.372) (size 0.6) (drill 0.3) (layers "F.Cu" "B.Cu") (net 12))
 (segment (start 130.153 103.547) (end 129.391 103.547) (width 0.2) (layer "B.Cu") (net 12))
 (segment (start 133.074 100.626) (end 130.153 103.547) (width 0.2) (layer "B.Cu") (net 12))
 (segment (start 133.074 100.372) (end 133.074 100.626) (width 0.2) (layer "B.Cu") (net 12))
 (segment (start 129.391 104.1058) (end 129.391 108.627) (width 0.2) (layer "F.Cu") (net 14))
 (segment (start 130.5848 102.912) (end 129.391 104.1058) (width 0.2) (layer "F.Cu") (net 14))
 (segment (start 131.296 102.912) (end 130.5848 102.912) (width 0.2) (layer "F.Cu") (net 14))
 (via (at 129.391 108.627) (size 0.6) (drill 0.3) (layers "F.Cu" "B.Cu") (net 14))
 (segment (start 143.326 95.292) (end 144.631 93.987) (width 0.2) (layer "F.Cu") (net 25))
 (segment (start 142.726 95.292) (end 143.326 95.292) (width 0.2) (layer "F.Cu") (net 25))
 (segment (start 144.631 93.987) (end 144.631 93.387) (width 0.2) (layer "F.Cu") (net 25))
 (via (at 144.631 93.387) (size 0.6) (drill 0.3) (layers "F.Cu" "B.Cu") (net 25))
 (segment (start 130.5848 95.292) (end 129.391 94.0982) (width 0.2) (layer "F.Cu") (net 8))
 (segment (start 131.296 95.292) (end 130.5848 95.292) (width 0.2) (layer "F.Cu") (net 8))
 (segment (start 129.391 94.0982) (end 129.391 93.387) (width 0.2) (layer "F.Cu") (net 8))
 (via (at 129.391 93.387) (size 0.6) (drill 0.3) (layers "F.Cu" "B.Cu") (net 8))
 (segment (start 131.296 105.452) (end 131.296 111.802) (width 0.2) (layer "F.Cu") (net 16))
 (segment (start 131.296 111.802) (end 129.391 113.707) (width 0.2) (layer "F.Cu") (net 16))
 (via (at 129.391 113.707) (size 0.6) (drill 0.3) (layers "F.Cu" "B.Cu") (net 16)))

